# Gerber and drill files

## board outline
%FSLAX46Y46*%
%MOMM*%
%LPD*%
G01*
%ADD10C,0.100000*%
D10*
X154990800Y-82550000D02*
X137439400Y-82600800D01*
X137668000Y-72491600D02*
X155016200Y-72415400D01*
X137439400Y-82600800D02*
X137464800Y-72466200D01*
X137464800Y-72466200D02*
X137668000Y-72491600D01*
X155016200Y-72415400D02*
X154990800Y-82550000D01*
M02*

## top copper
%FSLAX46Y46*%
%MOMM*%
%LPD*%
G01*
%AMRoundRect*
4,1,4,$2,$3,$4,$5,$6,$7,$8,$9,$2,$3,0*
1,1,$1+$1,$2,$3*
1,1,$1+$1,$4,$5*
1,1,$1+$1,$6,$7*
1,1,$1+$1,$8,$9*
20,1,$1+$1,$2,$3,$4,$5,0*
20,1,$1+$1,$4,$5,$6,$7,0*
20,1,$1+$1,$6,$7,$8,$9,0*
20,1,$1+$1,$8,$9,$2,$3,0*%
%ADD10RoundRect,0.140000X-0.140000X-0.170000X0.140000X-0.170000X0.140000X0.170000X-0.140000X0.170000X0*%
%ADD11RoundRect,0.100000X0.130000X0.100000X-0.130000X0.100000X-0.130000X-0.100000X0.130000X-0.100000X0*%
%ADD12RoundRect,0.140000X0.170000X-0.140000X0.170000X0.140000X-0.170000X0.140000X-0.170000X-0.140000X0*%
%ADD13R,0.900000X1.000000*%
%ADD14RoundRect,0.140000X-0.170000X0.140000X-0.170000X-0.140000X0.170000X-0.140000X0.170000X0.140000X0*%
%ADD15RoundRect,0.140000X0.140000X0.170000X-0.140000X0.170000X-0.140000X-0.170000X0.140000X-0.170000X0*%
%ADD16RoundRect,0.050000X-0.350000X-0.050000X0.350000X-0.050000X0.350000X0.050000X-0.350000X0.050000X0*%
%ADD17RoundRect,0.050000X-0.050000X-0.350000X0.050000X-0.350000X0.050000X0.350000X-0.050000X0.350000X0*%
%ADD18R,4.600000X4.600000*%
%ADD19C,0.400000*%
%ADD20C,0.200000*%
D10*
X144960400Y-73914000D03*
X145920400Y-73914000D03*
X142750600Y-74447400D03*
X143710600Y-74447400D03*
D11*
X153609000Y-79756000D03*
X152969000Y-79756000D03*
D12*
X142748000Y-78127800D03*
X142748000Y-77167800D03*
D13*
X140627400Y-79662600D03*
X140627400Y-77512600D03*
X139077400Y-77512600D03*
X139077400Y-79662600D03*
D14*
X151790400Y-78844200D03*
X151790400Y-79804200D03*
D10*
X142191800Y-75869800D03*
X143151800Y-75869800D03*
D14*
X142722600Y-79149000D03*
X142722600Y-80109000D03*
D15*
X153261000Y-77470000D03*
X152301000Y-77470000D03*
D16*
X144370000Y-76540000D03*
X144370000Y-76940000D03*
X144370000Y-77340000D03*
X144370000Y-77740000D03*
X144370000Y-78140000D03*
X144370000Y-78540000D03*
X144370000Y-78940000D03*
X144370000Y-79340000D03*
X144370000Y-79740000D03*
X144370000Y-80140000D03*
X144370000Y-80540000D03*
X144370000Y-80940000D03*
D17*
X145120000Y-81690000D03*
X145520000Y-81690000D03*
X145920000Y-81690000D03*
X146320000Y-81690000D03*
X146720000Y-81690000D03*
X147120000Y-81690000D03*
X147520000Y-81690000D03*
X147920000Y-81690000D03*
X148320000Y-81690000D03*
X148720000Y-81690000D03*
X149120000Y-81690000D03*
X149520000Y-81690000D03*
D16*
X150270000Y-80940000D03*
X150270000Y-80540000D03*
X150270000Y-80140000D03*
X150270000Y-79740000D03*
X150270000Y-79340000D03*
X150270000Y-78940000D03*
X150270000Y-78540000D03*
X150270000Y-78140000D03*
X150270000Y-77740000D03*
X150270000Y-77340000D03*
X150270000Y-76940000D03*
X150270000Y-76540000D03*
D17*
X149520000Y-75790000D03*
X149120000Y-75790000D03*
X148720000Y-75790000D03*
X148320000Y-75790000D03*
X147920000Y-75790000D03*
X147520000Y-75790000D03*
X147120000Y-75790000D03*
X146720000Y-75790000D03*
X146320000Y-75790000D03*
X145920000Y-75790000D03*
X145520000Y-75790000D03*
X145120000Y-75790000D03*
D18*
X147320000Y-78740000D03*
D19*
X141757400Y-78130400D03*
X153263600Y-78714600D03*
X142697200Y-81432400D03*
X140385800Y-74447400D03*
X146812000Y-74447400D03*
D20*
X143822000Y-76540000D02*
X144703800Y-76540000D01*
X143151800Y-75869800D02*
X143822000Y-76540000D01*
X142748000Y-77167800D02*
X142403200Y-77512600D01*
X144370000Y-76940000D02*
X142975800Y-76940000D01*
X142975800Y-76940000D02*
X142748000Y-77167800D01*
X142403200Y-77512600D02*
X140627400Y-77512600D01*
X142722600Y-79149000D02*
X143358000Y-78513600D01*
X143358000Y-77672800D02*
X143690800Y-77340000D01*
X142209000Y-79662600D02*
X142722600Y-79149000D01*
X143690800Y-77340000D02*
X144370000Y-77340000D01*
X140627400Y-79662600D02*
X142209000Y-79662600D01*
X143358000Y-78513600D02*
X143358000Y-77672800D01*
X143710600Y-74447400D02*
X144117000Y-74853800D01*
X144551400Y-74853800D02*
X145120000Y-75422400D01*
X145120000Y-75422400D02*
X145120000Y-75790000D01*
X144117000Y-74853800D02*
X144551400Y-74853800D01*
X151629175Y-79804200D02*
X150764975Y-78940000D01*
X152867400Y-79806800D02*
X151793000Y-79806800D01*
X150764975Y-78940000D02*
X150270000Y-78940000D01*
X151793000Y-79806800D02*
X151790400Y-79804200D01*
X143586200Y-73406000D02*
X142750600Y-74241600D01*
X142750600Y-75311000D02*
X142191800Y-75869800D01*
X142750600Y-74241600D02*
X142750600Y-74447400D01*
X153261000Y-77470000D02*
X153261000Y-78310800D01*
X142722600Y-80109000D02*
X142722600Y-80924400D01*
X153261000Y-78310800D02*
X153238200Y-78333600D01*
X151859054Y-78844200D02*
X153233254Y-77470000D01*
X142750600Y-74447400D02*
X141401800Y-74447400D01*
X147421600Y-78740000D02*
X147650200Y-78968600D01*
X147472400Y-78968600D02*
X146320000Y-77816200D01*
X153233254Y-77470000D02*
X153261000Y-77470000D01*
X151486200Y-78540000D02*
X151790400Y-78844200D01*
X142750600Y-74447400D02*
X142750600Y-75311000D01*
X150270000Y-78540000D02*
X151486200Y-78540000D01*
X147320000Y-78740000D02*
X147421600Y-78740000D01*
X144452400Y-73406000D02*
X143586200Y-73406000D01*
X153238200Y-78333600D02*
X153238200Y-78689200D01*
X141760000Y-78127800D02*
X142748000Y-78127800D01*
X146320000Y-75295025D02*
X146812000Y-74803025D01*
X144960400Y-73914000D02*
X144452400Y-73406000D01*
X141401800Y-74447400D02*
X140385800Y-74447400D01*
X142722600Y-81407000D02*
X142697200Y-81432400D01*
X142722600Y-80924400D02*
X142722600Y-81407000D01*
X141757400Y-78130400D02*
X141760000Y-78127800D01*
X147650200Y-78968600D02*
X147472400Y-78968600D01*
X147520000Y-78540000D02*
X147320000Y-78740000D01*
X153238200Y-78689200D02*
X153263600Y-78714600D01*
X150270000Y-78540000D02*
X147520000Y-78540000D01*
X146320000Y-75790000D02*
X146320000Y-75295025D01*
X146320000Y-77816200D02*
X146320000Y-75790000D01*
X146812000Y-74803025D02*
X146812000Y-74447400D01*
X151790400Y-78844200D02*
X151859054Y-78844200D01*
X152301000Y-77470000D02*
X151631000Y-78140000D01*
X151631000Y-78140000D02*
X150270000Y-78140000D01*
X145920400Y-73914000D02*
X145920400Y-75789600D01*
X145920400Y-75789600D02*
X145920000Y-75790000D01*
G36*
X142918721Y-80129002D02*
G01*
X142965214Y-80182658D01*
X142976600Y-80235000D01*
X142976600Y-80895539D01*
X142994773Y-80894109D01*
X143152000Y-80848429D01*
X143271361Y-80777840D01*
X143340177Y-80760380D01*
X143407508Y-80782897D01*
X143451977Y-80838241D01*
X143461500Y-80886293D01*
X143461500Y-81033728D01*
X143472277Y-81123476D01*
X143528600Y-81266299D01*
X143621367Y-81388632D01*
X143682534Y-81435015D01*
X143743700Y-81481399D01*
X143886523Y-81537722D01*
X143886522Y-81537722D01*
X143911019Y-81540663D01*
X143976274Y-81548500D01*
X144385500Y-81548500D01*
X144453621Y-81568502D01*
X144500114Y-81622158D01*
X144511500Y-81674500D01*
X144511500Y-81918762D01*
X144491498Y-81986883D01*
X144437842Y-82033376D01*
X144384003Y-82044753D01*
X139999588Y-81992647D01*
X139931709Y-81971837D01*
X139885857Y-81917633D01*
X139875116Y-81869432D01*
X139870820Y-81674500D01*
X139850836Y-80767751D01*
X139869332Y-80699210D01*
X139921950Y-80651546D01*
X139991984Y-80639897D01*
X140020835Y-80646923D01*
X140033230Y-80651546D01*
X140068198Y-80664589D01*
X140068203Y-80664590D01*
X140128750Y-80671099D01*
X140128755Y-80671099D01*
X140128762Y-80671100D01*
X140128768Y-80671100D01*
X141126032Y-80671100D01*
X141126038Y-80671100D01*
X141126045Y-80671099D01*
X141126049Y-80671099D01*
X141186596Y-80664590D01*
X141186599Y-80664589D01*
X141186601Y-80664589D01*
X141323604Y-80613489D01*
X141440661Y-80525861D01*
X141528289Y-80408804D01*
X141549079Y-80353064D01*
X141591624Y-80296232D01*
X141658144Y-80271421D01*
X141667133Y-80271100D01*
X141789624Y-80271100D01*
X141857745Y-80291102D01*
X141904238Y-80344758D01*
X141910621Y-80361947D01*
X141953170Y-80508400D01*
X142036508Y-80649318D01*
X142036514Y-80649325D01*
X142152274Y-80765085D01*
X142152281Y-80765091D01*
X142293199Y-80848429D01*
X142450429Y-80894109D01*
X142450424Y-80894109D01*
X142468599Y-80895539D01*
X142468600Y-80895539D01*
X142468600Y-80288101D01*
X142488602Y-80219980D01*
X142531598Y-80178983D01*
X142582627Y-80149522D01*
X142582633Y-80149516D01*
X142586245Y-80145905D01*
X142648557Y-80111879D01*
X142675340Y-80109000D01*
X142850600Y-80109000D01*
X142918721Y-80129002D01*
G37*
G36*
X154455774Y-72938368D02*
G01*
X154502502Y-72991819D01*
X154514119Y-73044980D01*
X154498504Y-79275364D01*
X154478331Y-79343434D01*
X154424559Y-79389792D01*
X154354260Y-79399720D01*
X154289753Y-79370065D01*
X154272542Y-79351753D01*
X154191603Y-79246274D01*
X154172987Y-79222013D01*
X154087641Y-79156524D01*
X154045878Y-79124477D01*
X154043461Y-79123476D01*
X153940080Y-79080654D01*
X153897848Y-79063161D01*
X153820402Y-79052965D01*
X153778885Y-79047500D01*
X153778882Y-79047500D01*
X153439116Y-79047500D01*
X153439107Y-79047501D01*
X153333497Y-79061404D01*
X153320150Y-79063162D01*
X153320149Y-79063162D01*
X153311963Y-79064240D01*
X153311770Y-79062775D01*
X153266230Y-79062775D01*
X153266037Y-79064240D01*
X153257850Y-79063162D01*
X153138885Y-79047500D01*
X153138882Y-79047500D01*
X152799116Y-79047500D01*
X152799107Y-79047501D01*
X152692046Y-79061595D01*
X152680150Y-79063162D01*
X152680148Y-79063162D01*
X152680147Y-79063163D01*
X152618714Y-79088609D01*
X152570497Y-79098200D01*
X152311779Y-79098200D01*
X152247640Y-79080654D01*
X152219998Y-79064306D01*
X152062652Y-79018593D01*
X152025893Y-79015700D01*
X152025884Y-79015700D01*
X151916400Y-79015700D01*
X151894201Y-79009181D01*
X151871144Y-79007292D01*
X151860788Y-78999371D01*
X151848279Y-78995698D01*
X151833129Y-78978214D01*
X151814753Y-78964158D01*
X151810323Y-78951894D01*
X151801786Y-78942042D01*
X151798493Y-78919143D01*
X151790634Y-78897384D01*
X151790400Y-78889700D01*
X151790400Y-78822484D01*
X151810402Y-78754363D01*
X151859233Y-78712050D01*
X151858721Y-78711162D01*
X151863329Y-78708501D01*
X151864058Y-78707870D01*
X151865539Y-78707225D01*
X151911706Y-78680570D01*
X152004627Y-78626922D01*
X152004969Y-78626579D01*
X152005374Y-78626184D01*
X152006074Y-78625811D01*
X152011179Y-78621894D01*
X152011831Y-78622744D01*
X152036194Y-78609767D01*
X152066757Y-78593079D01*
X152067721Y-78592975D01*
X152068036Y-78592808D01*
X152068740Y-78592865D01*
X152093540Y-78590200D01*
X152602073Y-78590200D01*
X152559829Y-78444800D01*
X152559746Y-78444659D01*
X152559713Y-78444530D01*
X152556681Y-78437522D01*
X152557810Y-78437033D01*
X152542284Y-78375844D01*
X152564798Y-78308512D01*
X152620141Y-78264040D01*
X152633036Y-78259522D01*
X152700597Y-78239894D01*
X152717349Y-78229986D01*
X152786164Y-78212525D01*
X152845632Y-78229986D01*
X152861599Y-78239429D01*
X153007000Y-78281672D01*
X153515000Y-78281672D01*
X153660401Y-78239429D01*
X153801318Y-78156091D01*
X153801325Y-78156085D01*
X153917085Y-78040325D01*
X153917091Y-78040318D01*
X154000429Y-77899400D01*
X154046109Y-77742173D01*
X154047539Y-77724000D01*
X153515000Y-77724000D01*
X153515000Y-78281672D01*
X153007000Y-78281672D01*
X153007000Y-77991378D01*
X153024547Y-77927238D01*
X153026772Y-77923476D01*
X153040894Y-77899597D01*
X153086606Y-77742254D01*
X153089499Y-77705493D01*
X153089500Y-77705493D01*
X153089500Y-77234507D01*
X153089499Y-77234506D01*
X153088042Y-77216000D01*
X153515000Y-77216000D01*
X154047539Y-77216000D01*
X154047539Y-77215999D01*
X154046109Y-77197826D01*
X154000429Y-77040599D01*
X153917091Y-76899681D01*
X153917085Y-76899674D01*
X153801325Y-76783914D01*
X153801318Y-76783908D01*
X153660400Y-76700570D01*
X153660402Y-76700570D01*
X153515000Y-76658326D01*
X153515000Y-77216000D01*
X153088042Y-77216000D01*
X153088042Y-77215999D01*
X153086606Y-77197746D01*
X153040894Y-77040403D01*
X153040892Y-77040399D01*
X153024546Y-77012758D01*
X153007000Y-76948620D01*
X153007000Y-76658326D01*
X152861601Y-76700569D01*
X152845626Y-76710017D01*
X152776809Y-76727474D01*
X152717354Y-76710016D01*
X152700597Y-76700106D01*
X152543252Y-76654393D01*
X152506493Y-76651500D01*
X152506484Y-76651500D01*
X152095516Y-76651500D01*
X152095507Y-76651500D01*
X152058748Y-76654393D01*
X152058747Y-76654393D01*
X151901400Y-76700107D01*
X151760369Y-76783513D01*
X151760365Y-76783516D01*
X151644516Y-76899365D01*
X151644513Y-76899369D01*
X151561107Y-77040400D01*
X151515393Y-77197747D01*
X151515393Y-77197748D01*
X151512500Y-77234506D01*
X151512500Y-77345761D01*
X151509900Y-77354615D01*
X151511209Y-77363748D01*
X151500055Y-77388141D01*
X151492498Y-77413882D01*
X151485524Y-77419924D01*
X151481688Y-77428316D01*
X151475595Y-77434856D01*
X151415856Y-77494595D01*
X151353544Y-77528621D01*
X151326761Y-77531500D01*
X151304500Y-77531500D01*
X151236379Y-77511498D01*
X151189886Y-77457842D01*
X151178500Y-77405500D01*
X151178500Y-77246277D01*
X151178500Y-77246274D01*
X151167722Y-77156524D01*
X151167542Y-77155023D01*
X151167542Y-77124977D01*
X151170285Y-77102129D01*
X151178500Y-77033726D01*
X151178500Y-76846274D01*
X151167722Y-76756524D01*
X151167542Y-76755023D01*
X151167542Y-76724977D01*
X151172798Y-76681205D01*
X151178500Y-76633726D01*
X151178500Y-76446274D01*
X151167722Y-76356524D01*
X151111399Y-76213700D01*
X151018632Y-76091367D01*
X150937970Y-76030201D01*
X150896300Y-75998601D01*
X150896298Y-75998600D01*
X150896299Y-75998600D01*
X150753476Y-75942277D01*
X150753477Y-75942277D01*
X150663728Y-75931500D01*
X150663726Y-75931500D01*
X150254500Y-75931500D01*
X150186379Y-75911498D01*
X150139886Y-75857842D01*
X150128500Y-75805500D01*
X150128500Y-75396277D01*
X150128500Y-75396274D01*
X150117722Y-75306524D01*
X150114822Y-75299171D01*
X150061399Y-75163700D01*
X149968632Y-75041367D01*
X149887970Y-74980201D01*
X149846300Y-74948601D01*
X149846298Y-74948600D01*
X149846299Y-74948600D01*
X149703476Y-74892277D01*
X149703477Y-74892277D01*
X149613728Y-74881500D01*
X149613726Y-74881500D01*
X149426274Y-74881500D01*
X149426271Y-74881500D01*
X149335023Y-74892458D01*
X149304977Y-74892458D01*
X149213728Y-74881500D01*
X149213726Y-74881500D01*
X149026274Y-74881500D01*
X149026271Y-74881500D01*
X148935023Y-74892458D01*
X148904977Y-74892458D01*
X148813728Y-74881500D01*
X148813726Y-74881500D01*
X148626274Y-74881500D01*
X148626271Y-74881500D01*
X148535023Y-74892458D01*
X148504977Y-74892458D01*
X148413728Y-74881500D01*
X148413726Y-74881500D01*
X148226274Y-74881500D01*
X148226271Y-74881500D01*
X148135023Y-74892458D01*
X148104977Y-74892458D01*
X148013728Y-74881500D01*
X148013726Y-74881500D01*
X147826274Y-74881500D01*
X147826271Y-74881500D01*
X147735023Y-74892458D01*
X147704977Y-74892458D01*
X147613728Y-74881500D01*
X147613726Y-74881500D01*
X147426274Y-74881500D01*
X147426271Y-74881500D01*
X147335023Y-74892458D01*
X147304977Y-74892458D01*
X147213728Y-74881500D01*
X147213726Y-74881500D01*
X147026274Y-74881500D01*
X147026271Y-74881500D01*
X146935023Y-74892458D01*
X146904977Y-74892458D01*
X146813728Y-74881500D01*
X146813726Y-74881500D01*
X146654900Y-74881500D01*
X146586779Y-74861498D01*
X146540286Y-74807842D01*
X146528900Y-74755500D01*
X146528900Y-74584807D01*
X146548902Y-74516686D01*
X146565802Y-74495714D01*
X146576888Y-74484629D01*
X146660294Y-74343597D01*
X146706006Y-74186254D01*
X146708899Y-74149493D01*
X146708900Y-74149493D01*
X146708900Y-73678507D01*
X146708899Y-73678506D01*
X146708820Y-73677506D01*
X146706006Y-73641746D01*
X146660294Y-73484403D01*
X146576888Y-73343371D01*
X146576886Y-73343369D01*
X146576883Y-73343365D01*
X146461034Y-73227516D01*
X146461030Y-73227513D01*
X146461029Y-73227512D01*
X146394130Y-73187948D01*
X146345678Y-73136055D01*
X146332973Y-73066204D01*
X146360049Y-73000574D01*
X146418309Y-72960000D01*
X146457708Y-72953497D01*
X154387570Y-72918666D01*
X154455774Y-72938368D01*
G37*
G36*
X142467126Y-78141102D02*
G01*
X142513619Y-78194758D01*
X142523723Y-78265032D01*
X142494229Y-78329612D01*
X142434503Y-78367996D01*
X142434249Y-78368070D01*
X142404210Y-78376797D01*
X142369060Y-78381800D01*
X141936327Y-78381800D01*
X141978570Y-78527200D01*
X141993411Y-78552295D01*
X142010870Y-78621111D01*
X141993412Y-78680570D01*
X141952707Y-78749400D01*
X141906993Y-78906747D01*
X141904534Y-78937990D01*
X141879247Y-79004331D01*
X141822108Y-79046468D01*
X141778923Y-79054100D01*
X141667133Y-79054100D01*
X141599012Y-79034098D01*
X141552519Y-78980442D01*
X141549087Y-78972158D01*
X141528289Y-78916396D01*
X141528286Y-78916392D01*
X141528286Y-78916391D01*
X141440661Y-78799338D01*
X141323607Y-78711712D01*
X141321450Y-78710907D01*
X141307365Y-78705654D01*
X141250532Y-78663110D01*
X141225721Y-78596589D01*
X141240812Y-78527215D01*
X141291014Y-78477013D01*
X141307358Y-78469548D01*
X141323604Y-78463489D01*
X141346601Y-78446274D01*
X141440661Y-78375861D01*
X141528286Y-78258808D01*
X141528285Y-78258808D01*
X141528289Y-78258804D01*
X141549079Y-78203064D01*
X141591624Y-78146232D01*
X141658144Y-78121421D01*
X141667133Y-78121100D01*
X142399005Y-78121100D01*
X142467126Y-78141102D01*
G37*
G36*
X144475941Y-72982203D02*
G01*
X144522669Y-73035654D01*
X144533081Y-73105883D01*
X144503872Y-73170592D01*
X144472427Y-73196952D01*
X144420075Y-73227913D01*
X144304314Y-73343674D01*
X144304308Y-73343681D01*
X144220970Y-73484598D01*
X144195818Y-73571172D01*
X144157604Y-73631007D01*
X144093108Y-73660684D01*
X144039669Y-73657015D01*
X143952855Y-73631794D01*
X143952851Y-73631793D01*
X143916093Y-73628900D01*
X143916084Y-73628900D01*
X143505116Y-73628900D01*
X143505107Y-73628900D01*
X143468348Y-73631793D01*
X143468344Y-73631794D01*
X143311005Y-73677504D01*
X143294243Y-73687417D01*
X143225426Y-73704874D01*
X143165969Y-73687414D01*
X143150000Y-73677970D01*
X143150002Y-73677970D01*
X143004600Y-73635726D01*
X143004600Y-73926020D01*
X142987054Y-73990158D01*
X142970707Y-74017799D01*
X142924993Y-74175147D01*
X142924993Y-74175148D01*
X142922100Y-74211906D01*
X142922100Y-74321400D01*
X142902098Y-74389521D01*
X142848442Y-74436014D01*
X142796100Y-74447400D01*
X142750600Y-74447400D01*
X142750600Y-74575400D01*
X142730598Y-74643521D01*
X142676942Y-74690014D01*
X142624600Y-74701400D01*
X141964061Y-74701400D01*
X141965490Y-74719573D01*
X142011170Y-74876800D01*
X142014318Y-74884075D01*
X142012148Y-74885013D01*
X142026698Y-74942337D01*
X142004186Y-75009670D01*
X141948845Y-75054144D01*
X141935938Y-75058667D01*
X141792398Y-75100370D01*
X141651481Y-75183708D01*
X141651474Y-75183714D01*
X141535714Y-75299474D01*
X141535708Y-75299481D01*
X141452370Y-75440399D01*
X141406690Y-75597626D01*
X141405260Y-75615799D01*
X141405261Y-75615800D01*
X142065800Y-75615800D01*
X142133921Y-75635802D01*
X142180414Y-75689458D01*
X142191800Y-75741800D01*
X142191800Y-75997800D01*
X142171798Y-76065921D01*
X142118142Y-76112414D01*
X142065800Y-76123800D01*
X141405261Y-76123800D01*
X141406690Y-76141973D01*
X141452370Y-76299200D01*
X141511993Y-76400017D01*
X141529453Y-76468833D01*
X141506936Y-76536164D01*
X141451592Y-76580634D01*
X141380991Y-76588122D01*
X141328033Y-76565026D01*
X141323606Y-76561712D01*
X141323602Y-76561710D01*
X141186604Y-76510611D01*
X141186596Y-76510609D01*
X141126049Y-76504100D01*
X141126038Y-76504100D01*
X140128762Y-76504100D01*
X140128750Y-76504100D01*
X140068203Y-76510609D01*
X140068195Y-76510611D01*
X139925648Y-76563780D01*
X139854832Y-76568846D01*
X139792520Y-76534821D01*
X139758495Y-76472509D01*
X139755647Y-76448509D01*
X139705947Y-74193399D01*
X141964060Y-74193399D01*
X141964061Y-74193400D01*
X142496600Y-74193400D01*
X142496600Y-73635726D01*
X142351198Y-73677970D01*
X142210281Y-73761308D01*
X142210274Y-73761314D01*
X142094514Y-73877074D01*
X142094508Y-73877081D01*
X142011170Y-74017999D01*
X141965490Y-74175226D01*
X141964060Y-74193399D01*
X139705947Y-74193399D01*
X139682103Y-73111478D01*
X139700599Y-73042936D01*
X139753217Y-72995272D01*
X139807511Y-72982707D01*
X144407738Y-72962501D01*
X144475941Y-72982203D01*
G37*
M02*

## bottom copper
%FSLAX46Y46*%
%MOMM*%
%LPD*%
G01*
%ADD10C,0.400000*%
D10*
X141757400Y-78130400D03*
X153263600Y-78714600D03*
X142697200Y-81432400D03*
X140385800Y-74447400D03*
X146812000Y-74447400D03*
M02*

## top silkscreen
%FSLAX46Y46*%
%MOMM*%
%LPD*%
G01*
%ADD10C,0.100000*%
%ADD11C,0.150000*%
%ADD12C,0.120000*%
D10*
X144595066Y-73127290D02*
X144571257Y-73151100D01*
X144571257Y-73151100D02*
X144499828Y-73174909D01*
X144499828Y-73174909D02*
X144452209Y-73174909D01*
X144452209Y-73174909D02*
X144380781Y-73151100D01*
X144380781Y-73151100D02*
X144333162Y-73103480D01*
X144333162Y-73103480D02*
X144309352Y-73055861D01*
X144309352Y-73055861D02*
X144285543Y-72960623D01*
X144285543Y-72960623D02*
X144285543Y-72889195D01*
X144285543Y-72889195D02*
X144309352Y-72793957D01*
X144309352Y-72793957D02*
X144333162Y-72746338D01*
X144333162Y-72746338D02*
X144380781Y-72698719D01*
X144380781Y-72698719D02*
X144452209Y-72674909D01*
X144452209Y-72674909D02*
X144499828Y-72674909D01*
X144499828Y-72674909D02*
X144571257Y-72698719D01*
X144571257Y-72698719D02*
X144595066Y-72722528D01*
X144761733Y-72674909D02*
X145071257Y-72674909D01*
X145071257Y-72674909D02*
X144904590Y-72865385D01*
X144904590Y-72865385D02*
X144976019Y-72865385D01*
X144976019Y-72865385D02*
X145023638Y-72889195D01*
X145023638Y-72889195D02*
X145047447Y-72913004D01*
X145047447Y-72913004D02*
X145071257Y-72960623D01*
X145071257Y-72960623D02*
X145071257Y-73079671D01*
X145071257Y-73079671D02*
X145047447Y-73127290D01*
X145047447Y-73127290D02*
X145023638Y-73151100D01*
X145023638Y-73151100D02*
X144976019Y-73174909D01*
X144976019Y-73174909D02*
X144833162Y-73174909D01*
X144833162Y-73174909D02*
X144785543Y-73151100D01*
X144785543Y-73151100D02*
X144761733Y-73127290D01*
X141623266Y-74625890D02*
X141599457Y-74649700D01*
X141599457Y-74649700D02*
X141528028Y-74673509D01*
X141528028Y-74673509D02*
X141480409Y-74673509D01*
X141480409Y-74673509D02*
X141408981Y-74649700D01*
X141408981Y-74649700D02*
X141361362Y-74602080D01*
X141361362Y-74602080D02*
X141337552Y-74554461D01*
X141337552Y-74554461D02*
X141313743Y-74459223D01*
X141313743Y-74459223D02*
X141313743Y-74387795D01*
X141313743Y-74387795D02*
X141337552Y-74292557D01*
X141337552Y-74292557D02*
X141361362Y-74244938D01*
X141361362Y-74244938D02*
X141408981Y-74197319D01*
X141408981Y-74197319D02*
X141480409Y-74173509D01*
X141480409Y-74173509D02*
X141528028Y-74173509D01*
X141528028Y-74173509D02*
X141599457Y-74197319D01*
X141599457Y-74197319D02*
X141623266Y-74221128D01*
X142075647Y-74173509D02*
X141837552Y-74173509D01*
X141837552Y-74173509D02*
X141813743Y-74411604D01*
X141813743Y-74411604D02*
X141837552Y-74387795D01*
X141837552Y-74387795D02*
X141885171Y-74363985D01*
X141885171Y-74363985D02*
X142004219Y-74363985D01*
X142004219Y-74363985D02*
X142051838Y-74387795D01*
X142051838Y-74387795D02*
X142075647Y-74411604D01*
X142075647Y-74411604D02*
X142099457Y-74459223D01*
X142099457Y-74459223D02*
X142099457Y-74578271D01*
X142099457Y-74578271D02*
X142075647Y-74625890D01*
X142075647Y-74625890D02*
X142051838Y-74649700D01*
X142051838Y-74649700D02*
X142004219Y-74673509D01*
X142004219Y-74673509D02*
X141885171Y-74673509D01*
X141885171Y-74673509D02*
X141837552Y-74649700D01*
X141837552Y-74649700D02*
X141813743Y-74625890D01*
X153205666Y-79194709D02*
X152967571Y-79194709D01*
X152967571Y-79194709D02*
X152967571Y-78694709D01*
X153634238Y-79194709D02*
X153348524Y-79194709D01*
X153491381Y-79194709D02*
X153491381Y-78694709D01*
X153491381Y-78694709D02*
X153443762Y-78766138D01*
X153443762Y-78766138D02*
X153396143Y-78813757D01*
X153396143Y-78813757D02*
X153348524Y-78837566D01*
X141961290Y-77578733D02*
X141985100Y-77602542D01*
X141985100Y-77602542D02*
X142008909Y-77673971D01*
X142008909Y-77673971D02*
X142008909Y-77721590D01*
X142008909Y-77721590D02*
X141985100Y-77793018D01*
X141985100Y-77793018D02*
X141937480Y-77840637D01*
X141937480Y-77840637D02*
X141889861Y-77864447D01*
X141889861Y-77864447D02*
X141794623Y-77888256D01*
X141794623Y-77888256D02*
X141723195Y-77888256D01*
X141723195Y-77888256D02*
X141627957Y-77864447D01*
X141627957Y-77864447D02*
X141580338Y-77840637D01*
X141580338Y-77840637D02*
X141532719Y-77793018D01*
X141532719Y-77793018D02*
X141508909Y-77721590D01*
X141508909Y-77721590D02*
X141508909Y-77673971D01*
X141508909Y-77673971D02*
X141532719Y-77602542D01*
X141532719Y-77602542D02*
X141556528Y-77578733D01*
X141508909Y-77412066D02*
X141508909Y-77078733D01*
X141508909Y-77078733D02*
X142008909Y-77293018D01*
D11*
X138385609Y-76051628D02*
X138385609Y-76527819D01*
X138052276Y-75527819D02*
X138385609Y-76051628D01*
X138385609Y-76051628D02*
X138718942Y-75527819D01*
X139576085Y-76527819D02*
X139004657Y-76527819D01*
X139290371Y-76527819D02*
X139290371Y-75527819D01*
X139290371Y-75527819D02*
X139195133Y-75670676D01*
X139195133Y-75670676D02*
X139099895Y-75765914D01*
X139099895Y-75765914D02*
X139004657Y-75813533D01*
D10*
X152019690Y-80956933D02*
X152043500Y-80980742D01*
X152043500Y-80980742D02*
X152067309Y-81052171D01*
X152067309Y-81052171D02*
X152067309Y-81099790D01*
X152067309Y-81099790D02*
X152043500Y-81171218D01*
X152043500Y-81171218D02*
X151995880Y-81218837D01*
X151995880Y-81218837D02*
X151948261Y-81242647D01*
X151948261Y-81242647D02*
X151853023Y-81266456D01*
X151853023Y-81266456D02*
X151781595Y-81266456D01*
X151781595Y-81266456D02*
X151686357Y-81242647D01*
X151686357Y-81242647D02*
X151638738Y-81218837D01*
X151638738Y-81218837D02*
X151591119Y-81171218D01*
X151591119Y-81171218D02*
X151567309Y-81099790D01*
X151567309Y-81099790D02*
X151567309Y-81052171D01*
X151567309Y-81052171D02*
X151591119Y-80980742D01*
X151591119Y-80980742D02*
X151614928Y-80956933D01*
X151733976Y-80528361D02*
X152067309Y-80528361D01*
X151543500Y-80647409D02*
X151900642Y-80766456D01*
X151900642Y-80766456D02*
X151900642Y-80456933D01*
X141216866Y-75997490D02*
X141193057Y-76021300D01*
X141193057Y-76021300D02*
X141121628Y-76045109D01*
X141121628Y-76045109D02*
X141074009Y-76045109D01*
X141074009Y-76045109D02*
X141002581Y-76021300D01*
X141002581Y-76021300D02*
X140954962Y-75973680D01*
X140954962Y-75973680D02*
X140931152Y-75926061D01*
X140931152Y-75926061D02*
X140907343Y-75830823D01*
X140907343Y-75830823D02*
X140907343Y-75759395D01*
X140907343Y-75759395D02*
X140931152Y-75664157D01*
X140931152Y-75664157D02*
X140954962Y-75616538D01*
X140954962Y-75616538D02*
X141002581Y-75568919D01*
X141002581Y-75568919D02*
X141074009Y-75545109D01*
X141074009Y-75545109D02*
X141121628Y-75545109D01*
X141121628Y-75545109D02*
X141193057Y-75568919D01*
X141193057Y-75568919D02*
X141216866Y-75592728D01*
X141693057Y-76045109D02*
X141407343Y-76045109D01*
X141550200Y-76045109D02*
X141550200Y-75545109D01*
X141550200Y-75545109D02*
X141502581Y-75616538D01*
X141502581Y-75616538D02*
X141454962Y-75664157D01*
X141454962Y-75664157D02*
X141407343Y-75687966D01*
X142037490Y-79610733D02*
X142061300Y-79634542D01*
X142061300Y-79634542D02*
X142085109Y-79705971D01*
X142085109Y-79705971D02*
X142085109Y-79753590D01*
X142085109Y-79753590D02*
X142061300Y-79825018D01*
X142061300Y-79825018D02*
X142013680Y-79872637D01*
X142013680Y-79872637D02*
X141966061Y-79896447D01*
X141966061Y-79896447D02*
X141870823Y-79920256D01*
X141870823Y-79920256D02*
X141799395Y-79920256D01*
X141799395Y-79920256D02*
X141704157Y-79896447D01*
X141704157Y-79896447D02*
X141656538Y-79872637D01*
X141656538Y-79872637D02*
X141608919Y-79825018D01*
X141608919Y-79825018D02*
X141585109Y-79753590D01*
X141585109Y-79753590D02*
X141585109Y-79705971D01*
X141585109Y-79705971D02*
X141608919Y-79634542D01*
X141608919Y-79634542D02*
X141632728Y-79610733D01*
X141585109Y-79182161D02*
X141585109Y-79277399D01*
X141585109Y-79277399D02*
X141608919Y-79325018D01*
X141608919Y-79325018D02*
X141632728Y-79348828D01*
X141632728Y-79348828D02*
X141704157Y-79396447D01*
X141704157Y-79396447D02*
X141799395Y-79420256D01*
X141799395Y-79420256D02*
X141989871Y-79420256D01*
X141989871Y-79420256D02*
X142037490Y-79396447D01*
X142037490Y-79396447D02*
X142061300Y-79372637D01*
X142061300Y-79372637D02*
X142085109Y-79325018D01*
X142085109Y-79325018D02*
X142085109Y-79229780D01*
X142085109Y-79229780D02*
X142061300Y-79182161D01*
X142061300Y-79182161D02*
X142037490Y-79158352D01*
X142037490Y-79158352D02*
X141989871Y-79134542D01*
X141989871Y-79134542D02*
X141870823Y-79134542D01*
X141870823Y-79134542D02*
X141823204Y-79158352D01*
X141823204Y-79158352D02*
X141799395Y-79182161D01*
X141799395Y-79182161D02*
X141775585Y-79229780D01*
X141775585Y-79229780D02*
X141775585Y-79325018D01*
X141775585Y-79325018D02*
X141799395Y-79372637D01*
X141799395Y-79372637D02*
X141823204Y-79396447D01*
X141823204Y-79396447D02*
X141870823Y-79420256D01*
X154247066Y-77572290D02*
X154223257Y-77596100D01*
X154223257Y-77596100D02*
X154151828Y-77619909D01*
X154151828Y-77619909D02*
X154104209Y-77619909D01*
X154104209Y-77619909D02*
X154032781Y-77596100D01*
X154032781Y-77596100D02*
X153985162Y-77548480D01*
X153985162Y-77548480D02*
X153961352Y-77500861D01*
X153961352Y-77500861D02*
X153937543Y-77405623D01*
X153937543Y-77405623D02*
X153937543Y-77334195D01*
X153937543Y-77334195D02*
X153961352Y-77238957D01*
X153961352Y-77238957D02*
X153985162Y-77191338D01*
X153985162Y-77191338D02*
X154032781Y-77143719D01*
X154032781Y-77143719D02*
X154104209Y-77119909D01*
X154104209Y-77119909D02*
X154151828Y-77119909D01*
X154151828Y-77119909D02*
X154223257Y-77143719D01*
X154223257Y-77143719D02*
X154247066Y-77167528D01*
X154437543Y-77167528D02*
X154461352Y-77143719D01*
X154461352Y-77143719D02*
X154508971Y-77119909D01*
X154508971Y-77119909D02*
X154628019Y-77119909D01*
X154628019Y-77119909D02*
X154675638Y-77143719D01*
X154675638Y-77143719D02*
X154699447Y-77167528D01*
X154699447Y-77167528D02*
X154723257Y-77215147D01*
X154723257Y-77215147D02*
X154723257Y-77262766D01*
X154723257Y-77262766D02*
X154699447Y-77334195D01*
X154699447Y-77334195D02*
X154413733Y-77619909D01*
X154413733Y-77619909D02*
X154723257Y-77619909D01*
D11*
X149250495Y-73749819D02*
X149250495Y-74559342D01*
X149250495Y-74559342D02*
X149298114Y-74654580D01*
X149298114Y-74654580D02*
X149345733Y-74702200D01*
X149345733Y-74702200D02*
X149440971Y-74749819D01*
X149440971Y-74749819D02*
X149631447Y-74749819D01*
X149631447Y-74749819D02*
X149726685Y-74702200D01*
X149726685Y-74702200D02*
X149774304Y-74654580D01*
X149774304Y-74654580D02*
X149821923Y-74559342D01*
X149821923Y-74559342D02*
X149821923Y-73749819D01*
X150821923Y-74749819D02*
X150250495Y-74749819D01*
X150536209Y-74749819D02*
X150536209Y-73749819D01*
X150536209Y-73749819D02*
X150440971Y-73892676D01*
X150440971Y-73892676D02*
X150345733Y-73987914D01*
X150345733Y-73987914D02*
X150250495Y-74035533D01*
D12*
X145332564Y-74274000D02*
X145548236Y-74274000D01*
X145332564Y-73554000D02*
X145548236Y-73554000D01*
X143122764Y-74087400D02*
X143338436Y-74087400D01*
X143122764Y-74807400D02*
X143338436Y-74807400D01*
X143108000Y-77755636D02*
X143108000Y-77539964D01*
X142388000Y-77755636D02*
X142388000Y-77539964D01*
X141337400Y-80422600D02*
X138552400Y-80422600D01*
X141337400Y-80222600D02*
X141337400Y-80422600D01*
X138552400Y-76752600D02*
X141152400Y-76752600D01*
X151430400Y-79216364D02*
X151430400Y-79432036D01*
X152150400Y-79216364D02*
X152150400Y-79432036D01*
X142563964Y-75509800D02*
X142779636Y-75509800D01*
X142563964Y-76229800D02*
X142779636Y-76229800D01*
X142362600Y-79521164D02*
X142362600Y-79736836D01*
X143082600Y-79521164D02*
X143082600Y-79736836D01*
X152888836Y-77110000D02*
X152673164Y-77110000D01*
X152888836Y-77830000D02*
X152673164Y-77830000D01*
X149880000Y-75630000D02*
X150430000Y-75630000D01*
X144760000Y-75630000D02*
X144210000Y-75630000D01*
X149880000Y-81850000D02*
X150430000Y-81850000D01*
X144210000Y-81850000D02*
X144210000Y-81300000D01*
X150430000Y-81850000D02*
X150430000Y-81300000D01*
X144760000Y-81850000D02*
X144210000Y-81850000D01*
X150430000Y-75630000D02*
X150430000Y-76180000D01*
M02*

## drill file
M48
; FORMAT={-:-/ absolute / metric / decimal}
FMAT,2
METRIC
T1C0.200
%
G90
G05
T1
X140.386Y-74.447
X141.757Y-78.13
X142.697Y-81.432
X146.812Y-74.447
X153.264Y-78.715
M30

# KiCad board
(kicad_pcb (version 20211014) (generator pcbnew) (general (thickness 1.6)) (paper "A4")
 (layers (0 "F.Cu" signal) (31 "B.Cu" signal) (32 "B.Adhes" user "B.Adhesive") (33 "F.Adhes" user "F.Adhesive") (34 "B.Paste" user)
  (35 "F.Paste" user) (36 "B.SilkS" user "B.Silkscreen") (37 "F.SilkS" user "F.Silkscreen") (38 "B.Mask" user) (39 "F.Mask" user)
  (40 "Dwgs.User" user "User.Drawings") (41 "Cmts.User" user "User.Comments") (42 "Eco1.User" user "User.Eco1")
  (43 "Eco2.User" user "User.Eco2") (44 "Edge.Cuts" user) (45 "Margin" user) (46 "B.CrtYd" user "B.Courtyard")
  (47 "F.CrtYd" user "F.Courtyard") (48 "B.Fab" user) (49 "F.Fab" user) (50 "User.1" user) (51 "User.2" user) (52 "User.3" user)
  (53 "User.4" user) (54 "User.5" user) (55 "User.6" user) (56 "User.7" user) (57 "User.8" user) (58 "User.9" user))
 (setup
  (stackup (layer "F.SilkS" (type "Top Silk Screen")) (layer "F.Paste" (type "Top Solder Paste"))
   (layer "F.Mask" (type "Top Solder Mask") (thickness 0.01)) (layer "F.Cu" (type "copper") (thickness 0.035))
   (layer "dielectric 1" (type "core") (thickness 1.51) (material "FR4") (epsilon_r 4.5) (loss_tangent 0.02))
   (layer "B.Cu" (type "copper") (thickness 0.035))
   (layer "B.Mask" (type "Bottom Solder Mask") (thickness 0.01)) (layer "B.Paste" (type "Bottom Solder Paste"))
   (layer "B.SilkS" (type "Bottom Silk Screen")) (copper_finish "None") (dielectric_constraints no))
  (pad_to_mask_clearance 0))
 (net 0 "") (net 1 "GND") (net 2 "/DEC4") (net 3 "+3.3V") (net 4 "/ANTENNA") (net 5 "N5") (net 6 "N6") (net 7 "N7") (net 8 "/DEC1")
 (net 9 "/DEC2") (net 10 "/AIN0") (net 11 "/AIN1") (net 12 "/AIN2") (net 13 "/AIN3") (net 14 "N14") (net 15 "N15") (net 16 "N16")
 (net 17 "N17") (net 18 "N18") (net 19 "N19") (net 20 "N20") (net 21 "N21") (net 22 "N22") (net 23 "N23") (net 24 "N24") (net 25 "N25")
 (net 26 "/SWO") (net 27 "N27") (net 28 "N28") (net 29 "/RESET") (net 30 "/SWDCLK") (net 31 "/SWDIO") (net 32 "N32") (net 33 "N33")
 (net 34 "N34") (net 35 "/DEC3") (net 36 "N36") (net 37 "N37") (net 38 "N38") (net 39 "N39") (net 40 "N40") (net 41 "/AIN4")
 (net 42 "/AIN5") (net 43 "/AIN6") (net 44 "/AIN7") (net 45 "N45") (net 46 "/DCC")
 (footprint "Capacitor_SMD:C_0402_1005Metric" (layer "F.Cu") (at 145.4404 73.914)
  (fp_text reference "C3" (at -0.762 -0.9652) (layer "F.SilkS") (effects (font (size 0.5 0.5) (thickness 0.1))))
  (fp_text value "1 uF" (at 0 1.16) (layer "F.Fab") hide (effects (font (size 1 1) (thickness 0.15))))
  (fp_line (start -0.107836 0.36) (end 0.107836 0.36) (layer "F.SilkS") (width 0.12))
  (fp_line (start -0.107836 -0.36) (end 0.107836 -0.36) (layer "F.SilkS") (width 0.12))
  (pad "1" smd roundrect (at -0.48 0) (size 0.56 0.62) (layers "F.Cu" "F.Paste" "F.Mask") (roundrect_rratio 0.25) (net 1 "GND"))
  (pad "2" smd roundrect (at 0.48 0) (size 0.56 0.62) (layers "F.Cu" "F.Paste" "F.Mask") (roundrect_rratio 0.25) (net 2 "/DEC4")))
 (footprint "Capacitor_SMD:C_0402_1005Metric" (layer "F.Cu") (at 143.2306 74.4474)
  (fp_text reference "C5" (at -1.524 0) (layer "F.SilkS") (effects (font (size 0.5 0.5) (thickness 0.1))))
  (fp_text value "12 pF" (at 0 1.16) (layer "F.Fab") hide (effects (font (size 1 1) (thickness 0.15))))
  (fp_line (start -0.107836 -0.36) (end 0.107836 -0.36) (layer "F.SilkS") (width 0.12))
  (fp_line (start -0.107836 0.36) (end 0.107836 0.36) (layer "F.SilkS") (width 0.12))
  (pad "1" smd roundrect (at -0.48 0) (size 0.56 0.62) (layers "F.Cu" "F.Paste" "F.Mask") (roundrect_rratio 0.25) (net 1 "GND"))
  (pad "2" smd roundrect (at 0.48 0) (size 0.56 0.62) (layers "F.Cu" "F.Paste" "F.Mask") (roundrect_rratio 0.25) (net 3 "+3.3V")))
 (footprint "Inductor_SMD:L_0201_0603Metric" (layer "F.Cu") (at 153.289 79.756 180)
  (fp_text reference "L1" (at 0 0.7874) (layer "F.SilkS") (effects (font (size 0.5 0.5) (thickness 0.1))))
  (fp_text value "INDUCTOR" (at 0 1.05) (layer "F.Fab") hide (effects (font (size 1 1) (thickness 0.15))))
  (pad "" smd roundrect (at -0.345 0 180) (size 0.318 0.36) (layers "F.Paste") (roundrect_rratio 0.25))
  (pad "" smd roundrect (at 0.345 0 180) (size 0.318 0.36) (layers "F.Paste") (roundrect_rratio 0.25))
  (pad "1" smd roundrect (at -0.32 0 180) (size 0.46 0.4) (layers "F.Cu" "F.Mask") (roundrect_rratio 0.25) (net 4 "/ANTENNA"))
  (pad "2" smd roundrect (at 0.32 0 180) (size 0.46 0.4) (layers "F.Cu" "F.Mask") (roundrect_rratio 0.25) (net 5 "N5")))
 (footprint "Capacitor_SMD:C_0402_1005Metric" (layer "F.Cu") (at 142.748 77.6478 90)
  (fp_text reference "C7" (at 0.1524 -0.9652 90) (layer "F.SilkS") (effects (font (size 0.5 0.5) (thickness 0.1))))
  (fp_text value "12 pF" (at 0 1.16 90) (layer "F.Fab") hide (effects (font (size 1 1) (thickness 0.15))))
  (fp_line (start -0.107836 0.36) (end 0.107836 0.36) (layer "F.SilkS") (width 0.12))
  (fp_line (start -0.107836 -0.36) (end 0.107836 -0.36) (layer "F.SilkS") (width 0.12))
  (pad "1" smd roundrect (at -0.48 0 90) (size 0.56 0.62) (layers "F.Cu" "F.Paste" "F.Mask") (roundrect_rratio 0.25) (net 1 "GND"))
  (pad "2" smd roundrect (at 0.48 0 90) (size 0.56 0.62) (layers "F.Cu" "F.Paste" "F.Mask") (roundrect_rratio 0.25) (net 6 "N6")))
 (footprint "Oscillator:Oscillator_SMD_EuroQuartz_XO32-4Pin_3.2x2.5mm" (layer "F.Cu") (at 139.8524 78.5876 180)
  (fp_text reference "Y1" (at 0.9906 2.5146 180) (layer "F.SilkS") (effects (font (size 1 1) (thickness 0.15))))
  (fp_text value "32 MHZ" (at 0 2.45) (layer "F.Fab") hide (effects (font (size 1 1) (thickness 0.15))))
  (fp_line (start -1.485 -1.835) (end 1.3 -1.835) (layer "F.SilkS") (width 0.12))
  (fp_line (start -1.485 -1.635) (end -1.485 -1.835) (layer "F.SilkS") (width 0.12))
  (fp_line (start 1.3 1.835) (end -1.3 1.835) (layer "F.SilkS") (width 0.12))
  (pad "1" smd rect (at -0.775 -1.075 90) (size 1 0.9) (layers "F.Cu" "F.Paste" "F.Mask") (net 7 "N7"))
  (pad "2" smd rect (at -0.775 1.075 90) (size 1 0.9) (layers "F.Cu" "F.Paste" "F.Mask") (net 6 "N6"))
  (pad "3" smd rect (at 0.775 1.075 90) (size 1 0.9) (layers "F.Cu" "F.Paste" "F.Mask"))
  (pad "4" smd rect (at 0.775 -1.075 90) (size 1 0.9) (layers "F.Cu" "F.Paste" "F.Mask")))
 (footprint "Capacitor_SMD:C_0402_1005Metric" (layer "F.Cu") (at 151.7904 79.3242 -90)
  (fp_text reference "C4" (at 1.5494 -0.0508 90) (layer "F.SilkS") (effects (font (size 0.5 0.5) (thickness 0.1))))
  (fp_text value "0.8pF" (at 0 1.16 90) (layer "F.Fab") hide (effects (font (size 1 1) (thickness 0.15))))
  (fp_line (start -0.107836 0.36) (end 0.107836 0.36) (layer "F.SilkS") (width 0.12))
  (fp_line (start -0.107836 -0.36) (end 0.107836 -0.36) (layer "F.SilkS") (width 0.12))
  (pad "1" smd roundrect (at -0.48 0 270) (size 0.56 0.62) (layers "F.Cu" "F.Paste" "F.Mask") (roundrect_rratio 0.25) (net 1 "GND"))
  (pad "2" smd roundrect (at 0.48 0 270) (size 0.56 0.62) (layers "F.Cu" "F.Paste" "F.Mask") (roundrect_rratio 0.25) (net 5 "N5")))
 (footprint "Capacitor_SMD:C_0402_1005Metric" (layer "F.Cu") (at 142.6718 75.8698)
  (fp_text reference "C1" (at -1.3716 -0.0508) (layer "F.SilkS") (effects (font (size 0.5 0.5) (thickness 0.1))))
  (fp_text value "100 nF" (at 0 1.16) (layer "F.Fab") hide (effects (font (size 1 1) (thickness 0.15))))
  (fp_line (start -0.107836 -0.36) (end 0.107836 -0.36) (layer "F.SilkS") (width 0.12))
  (fp_line (start -0.107836 0.36) (end 0.107836 0.36) (layer "F.SilkS") (width 0.12))
  (pad "1" smd roundrect (at -0.48 0) (size 0.56 0.62) (layers "F.Cu" "F.Paste" "F.Mask") (roundrect_rratio 0.25) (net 1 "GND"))
  (pad "2" smd roundrect (at 0.48 0) (size 0.56 0.62) (layers "F.Cu" "F.Paste" "F.Mask") (roundrect_rratio 0.25) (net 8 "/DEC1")))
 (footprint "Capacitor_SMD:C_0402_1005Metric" (layer "F.Cu") (at 142.7226 79.629 -90)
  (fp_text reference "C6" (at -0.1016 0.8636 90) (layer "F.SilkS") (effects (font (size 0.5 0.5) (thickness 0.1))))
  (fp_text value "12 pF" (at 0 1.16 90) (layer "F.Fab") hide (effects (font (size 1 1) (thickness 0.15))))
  (fp_line (start -0.107836 0.36) (end 0.107836 0.36) (layer "F.SilkS") (width 0.12))
  (fp_line (start -0.107836 -0.36) (end 0.107836 -0.36) (layer "F.SilkS") (width 0.12))
  (pad "1" smd roundrect (at -0.48 0 270) (size 0.56 0.62) (layers "F.Cu" "F.Paste" "F.Mask") (roundrect_rratio 0.25) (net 7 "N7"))
  (pad "2" smd roundrect (at 0.48 0 270) (size 0.56 0.62) (layers "F.Cu" "F.Paste" "F.Mask") (roundrect_rratio 0.25) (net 1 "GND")))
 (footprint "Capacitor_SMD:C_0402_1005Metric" (layer "F.Cu") (at 152.781 77.47 180)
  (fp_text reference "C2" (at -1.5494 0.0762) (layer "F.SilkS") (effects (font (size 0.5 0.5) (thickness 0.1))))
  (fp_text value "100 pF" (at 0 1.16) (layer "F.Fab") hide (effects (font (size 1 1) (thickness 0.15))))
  (fp_line (start -0.107836 0.36) (end 0.107836 0.36) (layer "F.SilkS") (width 0.12))
  (fp_line (start -0.107836 -0.36) (end 0.107836 -0.36) (layer "F.SilkS") (width 0.12))
  (pad "1" smd roundrect (at -0.48 0 180) (size 0.56 0.62) (layers "F.Cu" "F.Paste" "F.Mask") (roundrect_rratio 0.25) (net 1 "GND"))
  (pad "2" smd roundrect (at 0.48 0 180) (size 0.56 0.62) (layers "F.Cu" "F.Paste" "F.Mask") (roundrect_rratio 0.25) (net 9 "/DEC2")))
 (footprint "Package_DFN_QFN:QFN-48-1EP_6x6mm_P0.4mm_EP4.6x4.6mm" (layer "F.Cu") (at 147.32 78.74)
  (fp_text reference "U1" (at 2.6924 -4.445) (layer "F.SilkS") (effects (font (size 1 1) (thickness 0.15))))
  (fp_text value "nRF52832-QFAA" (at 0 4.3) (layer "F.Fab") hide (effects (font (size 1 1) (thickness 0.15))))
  (fp_line (start 2.56 -3.11) (end 3.11 -3.11) (layer "F.SilkS") (width 0.12))
  (fp_line (start -2.56 -3.11) (end -3.11 -3.11) (layer "F.SilkS") (width 0.12))
  (fp_line (start 2.56 3.11) (end 3.11 3.11) (layer "F.SilkS") (width 0.12))
  (fp_line (start -3.11 3.11) (end -3.11 2.56) (layer "F.SilkS") (width 0.12))
  (fp_line (start 3.11 3.11) (end 3.11 2.56) (layer "F.SilkS") (width 0.12))
  (fp_line (start -2.56 3.11) (end -3.11 3.11) (layer "F.SilkS") (width 0.12))
  (fp_line (start 3.11 -3.11) (end 3.11 -2.56) (layer "F.SilkS") (width 0.12))
  (pad "" smd roundrect (at 0 1.53) (size 1.24 1.24) (layers "F.Paste") (roundrect_rratio 0.201613))
  (pad "" smd roundrect (at 1.53 -1.53) (size 1.24 1.24) (layers "F.Paste") (roundrect_rratio 0.201613))
  (pad "" smd roundrect (at 1.53 0) (size 1.24 1.24) (layers "F.Paste") (roundrect_rratio 0.201613))
  (pad "" smd roundrect (at 0 0) (size 1.24 1.24) (layers "F.Paste") (roundrect_rratio 0.201613))
  (pad "" smd roundrect (at -1.53 0) (size 1.24 1.24) (layers "F.Paste") (roundrect_rratio 0.201613))
  (pad "" smd roundrect (at 1.53 1.53) (size 1.24 1.24) (layers "F.Paste") (roundrect_rratio 0.201613))
  (pad "" smd roundrect (at 0 -1.53) (size 1.24 1.24) (layers "F.Paste") (roundrect_rratio 0.201613))
  (pad "" smd roundrect (at -1.53 -1.53) (size 1.24 1.24) (layers "F.Paste") (roundrect_rratio 0.201613))
  (pad "" smd roundrect (at -1.53 1.53) (size 1.24 1.24) (layers "F.Paste") (roundrect_rratio 0.201613))
  (pad "1" smd roundrect (at -2.95 -2.2) (size 0.8 0.2) (layers "F.Cu" "F.Paste" "F.Mask") (roundrect_rratio 0.25) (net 8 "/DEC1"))
  (pad "2" smd roundrect (at -2.95 -1.8) (size 0.8 0.2) (layers "F.Cu" "F.Paste" "F.Mask") (roundrect_rratio 0.25) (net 6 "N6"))
  (pad "3" smd roundrect (at -2.95 -1.4) (size 0.8 0.2) (layers "F.Cu" "F.Paste" "F.Mask") (roundrect_rratio 0.25) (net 7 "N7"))
  (pad "4" smd roundrect (at -2.95 -1) (size 0.8 0.2) (layers "F.Cu" "F.Paste" "F.Mask") (roundrect_rratio 0.25) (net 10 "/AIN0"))
  (pad "5" smd roundrect (at -2.95 -0.6) (size 0.8 0.2) (layers "F.Cu" "F.Paste" "F.Mask") (roundrect_rratio 0.25) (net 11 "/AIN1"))
  (pad "6" smd roundrect (at -2.95 -0.2) (size 0.8 0.2) (layers "F.Cu" "F.Paste" "F.Mask") (roundrect_rratio 0.25) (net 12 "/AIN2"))
  (pad "7" smd roundrect (at -2.95 0.2) (size 0.8 0.2) (layers "F.Cu" "F.Paste" "F.Mask") (roundrect_rratio 0.25) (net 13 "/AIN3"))
  (pad "8" smd roundrect (at -2.95 0.6) (size 0.8 0.2) (layers "F.Cu" "F.Paste" "F.Mask") (roundrect_rratio 0.25) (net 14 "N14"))
  (pad "9" smd roundrect (at -2.95 1) (size 0.8 0.2) (layers "F.Cu" "F.Paste" "F.Mask") (roundrect_rratio 0.25) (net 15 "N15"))
  (pad "10" smd roundrect (at -2.95 1.4) (size 0.8 0.2) (layers "F.Cu" "F.Paste" "F.Mask") (roundrect_rratio 0.25) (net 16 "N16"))
  (pad "11" smd roundrect (at -2.95 1.8) (size 0.8 0.2) (layers "F.Cu" "F.Paste" "F.Mask") (roundrect_rratio 0.25) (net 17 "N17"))
  (pad "12" smd roundrect (at -2.95 2.2) (size 0.8 0.2) (layers "F.Cu" "F.Paste" "F.Mask") (roundrect_rratio 0.25) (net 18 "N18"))
  (pad "13" smd roundrect (at -2.2 2.95) (size 0.2 0.8) (layers "F.Cu" "F.Paste" "F.Mask") (roundrect_rratio 0.25) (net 3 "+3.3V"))
  (pad "14" smd roundrect (at -1.8 2.95) (size 0.2 0.8) (layers "F.Cu" "F.Paste" "F.Mask") (roundrect_rratio 0.25) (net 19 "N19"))
  (pad "15" smd roundrect (at -1.4 2.95) (size 0.2 0.8) (layers "F.Cu" "F.Paste" "F.Mask") (roundrect_rratio 0.25) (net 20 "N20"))
  (pad "16" smd roundrect (at -1 2.95) (size 0.2 0.8) (layers "F.Cu" "F.Paste" "F.Mask") (roundrect_rratio 0.25) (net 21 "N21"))
  (pad "17" smd roundrect (at -0.6 2.95) (size 0.2 0.8) (layers "F.Cu" "F.Paste" "F.Mask") (roundrect_rratio 0.25) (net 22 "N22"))
  (pad "18" smd roundrect (at -0.2 2.95) (size 0.2 0.8) (layers "F.Cu" "F.Paste" "F.Mask") (roundrect_rratio 0.25) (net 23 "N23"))
  (pad "19" smd roundrect (at 0.2 2.95) (size 0.2 0.8) (layers "F.Cu" "F.Paste" "F.Mask") (roundrect_rratio 0.25) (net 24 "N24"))
  (pad "20" smd roundrect (at 0.6 2.95) (size 0.2 0.8) (layers "F.Cu" "F.Paste" "F.Mask") (roundrect_rratio 0.25) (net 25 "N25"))
  (pad "21" smd roundrect (at 1 2.95) (size 0.2 0.8) (layers "F.Cu" "F.Paste" "F.Mask") (roundrect_rratio 0.25) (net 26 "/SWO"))
  (pad "22" smd roundrect (at 1.4 2.95) (size 0.2 0.8) (layers "F.Cu" "F.Paste" "F.Mask") (roundrect_rratio 0.25) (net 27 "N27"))
  (pad "23" smd roundrect (at 1.8 2.95) (size 0.2 0.8) (layers "F.Cu" "F.Paste" "F.Mask") (roundrect_rratio 0.25) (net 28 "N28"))
  (pad "24" smd roundrect (at 2.2 2.95) (size 0.2 0.8) (layers "F.Cu" "F.Paste" "F.Mask") (roundrect_rratio 0.25) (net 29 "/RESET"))
  (pad "25" smd roundrect (at 2.95 2.2) (size 0.8 0.2) (layers "F.Cu" "F.Paste" "F.Mask") (roundrect_rratio 0.25) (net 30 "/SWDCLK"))
  (pad "26" smd roundrect (at 2.95 1.8) (size 0.8 0.2) (layers "F.Cu" "F.Paste" "F.Mask") (roundrect_rratio 0.25) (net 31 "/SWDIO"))
  (pad "27" smd roundrect (at 2.95 1.4) (size 0.8 0.2) (layers "F.Cu" "F.Paste" "F.Mask") (roundrect_rratio 0.25) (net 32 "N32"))
  (pad "28" smd roundrect (at 2.95 1) (size 0.8 0.2) (layers "F.Cu" "F.Paste" "F.Mask") (roundrect_rratio 0.25) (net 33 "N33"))
  (pad "29" smd roundrect (at 2.95 0.6) (size 0.8 0.2) (layers "F.Cu" "F.Paste" "F.Mask") (roundrect_rratio 0.25) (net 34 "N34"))
  (pad "30" smd roundrect (at 2.95 0.2) (size 0.8 0.2) (layers "F.Cu" "F.Paste" "F.Mask") (roundrect_rratio 0.25) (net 5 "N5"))
  (pad "31" smd roundrect (at 2.95 -0.2) (size 0.8 0.2) (layers "F.Cu" "F.Paste" "F.Mask") (roundrect_rratio 0.25) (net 1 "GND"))
  (pad "32" smd roundrect (at 2.95 -0.6) (size 0.8 0.2) (layers "F.Cu" "F.Paste" "F.Mask") (roundrect_rratio 0.25) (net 9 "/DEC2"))
  (pad "33" smd roundrect (at 2.95 -1) (size 0.8 0.2) (layers "F.Cu" "F.Paste" "F.Mask") (roundrect_rratio 0.25) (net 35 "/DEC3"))
  (pad "34" smd roundrect (at 2.95 -1.4) (size 0.8 0.2) (layers "F.Cu" "F.Paste" "F.Mask") (roundrect_rratio 0.25) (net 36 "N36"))
  (pad "35" smd roundrect (at 2.95 -1.8) (size 0.8 0.2) (layers "F.Cu" "F.Paste" "F.Mask") (roundrect_rratio 0.25) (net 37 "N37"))
  (pad "36" smd roundrect (at 2.95 -2.2) (size 0.8 0.2) (layers "F.Cu" "F.Paste" "F.Mask") (roundrect_rratio 0.25) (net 3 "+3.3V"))
  (pad "37" smd roundrect (at 2.2 -2.95) (size 0.2 0.8) (layers "F.Cu" "F.Paste" "F.Mask") (roundrect_rratio 0.25) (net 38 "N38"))
  (pad "38" smd roundrect (at 1.8 -2.95) (size 0.2 0.8) (layers "F.Cu" "F.Paste" "F.Mask") (roundrect_rratio 0.25) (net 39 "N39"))
  (pad "39" smd roundrect (at 1.4 -2.95) (size 0.2 0.8) (layers "F.Cu" "F.Paste" "F.Mask") (roundrect_rratio 0.25) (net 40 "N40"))
  (pad "40" smd roundrect (at 1 -2.95) (size 0.2 0.8) (layers "F.Cu" "F.Paste" "F.Mask") (roundrect_rratio 0.25) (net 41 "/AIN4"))
  (pad "41" smd roundrect (at 0.6 -2.95) (size 0.2 0.8) (layers "F.Cu" "F.Paste" "F.Mask") (roundrect_rratio 0.25) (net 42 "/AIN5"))
  (pad "42" smd roundrect (at 0.2 -2.95) (size 0.2 0.8) (layers "F.Cu" "F.Paste" "F.Mask") (roundrect_rratio 0.25) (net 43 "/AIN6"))
  (pad "43" smd roundrect (at -0.2 -2.95) (size 0.2 0.8) (layers "F.Cu" "F.Paste" "F.Mask") (roundrect_rratio 0.25) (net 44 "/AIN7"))
  (pad "44" smd roundrect (at -0.6 -2.95) (size 0.2 0.8) (layers "F.Cu" "F.Paste" "F.Mask") (roundrect_rratio 0.25) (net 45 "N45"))
  (pad "45" smd roundrect (at -1 -2.95) (size 0.2 0.8) (layers "F.Cu" "F.Paste" "F.Mask") (roundrect_rratio 0.25) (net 1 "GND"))
  (pad "46" smd roundrect (at -1.4 -2.95) (size 0.2 0.8) (layers "F.Cu" "F.Paste" "F.Mask") (roundrect_rratio 0.25) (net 2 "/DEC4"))
  (pad "47" smd roundrect (at -1.8 -2.95) (size 0.2 0.8) (layers "F.Cu" "F.Paste" "F.Mask") (roundrect_rratio 0.25) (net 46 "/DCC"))
  (pad "48" smd roundrect (at -2.2 -2.95) (size 0.2 0.8) (layers "F.Cu" "F.Paste" "F.Mask") (roundrect_rratio 0.25) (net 3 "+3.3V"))
  (pad "49" smd rect (at 0 0) (size 4.6 4.6) (layers "F.Cu" "F.Mask") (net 1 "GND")))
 (gr_line (start 154.9908 82.55) (end 137.4394 82.6008) (layer "Edge.Cuts") (width 0.1))
 (gr_line (start 137.668 72.4916) (end 155.0162 72.4154) (layer "Edge.Cuts") (width 0.1))
 (gr_line (start 137.4394 82.6008) (end 137.4648 72.4662) (layer "Edge.Cuts") (width 0.1))
 (gr_line (start 137.4648 72.4662) (end 137.668 72.4916) (layer "Edge.Cuts") (width 0.1))
 (gr_line (start 155.0162 72.4154) (end 154.9908 82.55) (layer "Edge.Cuts") (width 0.1))
 (segment (start 143.822 76.54) (end 144.7038 76.54) (width 0.2) (layer "F.Cu") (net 8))
 (segment (start 143.1518 75.8698) (end 143.822 76.54) (width 0.2) (layer "F.Cu") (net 8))
 (segment (start 142.748 77.1678) (end 142.4032 77.5126) (width 0.2) (layer "F.Cu") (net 6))
 (segment (start 144.37 76.94) (end 142.9758 76.94) (width 0.2) (layer "F.Cu") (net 6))
 (segment (start 142.9758 76.94) (end 142.748 77.1678) (width 0.2) (layer "F.Cu") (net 6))
 (segment (start 142.4032 77.5126) (end 140.6274 77.5126) (width 0.2) (layer "F.Cu") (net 6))
 (segment (start 142.7226 79.149) (end 143.358 78.5136) (width 0.2) (layer "F.Cu") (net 7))
 (segment (start 143.358 77.6728) (end 143.6908 77.34) (width 0.2) (layer "F.Cu") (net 7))
 (segment (start 142.209 79.6626) (end 142.7226 79.149) (width 0.2) (layer "F.Cu") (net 7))
 (segment (start 143.6908 77.34) (end 144.37 77.34) (width 0.2) (layer "F.Cu") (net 7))
 (segment (start 140.6274 79.6626) (end 142.209 79.6626) (width 0.2) (layer "F.Cu") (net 7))
 (segment (start 143.358 78.5136) (end 143.358 77.6728) (width 0.2) (layer "F.Cu") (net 7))
 (segment (start 143.7106 74.4474) (end 144.117 74.8538) (width 0.2) (layer "F.Cu") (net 3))
 (segment (start 144.5514 74.8538) (end 145.12 75.4224) (width 0.2) (layer "F.Cu") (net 3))
 (segment (start 145.12 75.4224) (end 145.12 75.79) (width 0.2) (layer "F.Cu") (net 3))
 (segment (start 144.117 74.8538) (end 144.5514 74.8538) (width 0.2) (layer "F.Cu") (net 3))
 (segment (start 151.629175 79.8042) (end 150.764975 78.94) (width 0.2) (layer "F.Cu") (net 5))
 (segment (start 152.8674 79.8068) (end 151.793 79.8068) (width 0.2) (layer "F.Cu") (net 5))
 (segment (start 150.764975 78.94) (end 150.27 78.94) (width 0.2) (layer "F.Cu") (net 5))
 (segment (start 151.793 79.8068) (end 151.7904 79.8042) (width 0.2) (layer "F.Cu") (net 5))
 (segment (start 143.5862 73.406) (end 142.7506 74.2416) (width 0.2) (layer "F.Cu") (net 1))
 (segment (start 142.7506 75.311) (end 142.1918 75.8698) (width 0.2) (layer "F.Cu") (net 1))
 (segment (start 142.7506 74.2416) (end 142.7506 74.4474) (width 0.2) (layer "F.Cu") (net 1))
 (segment (start 153.261 77.47) (end 153.261 78.3108) (width 0.2) (layer "F.Cu") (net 1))
 (segment (start 142.7226 80.109) (end 142.7226 80.9244) (width 0.2) (layer "F.Cu") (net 1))
 (segment (start 153.261 78.3108) (end 153.2382 78.3336) (width 0.2) (layer "F.Cu") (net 1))
 (segment (start 151.859054 78.8442) (end 153.233254 77.47) (width 0.2) (layer "F.Cu") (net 1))
 (segment (start 142.7506 74.4474) (end 141.4018 74.4474) (width 0.2) (layer "F.Cu") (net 1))
 (segment (start 147.4216 78.74) (end 147.6502 78.9686) (width 0.2) (layer "F.Cu") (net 1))
 (segment (start 147.4724 78.9686) (end 146.32 77.8162) (width 0.2) (layer "F.Cu") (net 1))
 (segment (start 153.233254 77.47) (end 153.261 77.47) (width 0.2) (layer "F.Cu") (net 1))
 (segment (start 151.4862 78.54) (end 151.7904 78.8442) (width 0.2) (layer "F.Cu") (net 1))
 (segment (start 142.7506 74.4474) (end 142.7506 75.311) (width 0.2) (layer "F.Cu") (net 1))
 (segment (start 150.27 78.54) (end 151.4862 78.54) (width 0.2) (layer "F.Cu") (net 1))
 (segment (start 147.32 78.74) (end 147.4216 78.74) (width 0.2) (layer "F.Cu") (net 1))
 (segment (start 144.4524 73.406) (end 143.5862 73.406) (width 0.2) (layer "F.Cu") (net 1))
 (segment (start 153.2382 78.3336) (end 153.2382 78.6892) (width 0.2) (layer "F.Cu") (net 1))
 (segment (start 141.76 78.1278) (end 142.748 78.1278) (width 0.2) (layer "F.Cu") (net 1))
 (segment (start 146.32 75.295025) (end 146.812 74.803025) (width 0.2) (layer "F.Cu") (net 1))
 (segment (start 144.9604 73.914) (end 144.4524 73.406) (width 0.2) (layer "F.Cu") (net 1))
 (segment (start 141.4018 74.4474) (end 140.3858 74.4474) (width 0.2) (layer "F.Cu") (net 1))
 (segment (start 142.7226 81.407) (end 142.6972 81.4324) (width 0.2) (layer "F.Cu") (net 1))
 (segment (start 142.7226 80.9244) (end 142.7226 81.407) (width 0.2) (layer "F.Cu") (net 1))
 (segment (start 141.7574 78.1304) (end 141.76 78.1278) (width 0.2) (layer "F.Cu") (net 1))
 (segment (start 147.6502 78.9686) (end 147.4724 78.9686) (width 0.2) (layer "F.Cu") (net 1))
 (segment (start 147.52 78.54) (end 147.32 78.74) (width 0.2) (layer "F.Cu") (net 1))
 (segment (start 153.2382 78.6892) (end 153.2636 78.7146) (width 0.2) (layer "F.Cu") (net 1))
 (segment (start 150.27 78.54) (end 147.52 78.54) (width 0.2) (layer "F.Cu") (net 1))
 (segment (start 146.32 75.79) (end 146.32 75.295025) (width 0.2) (layer "F.Cu") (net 1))
 (segment (start 146.32 77.8162) (end 146.32 75.79) (width 0.2) (layer "F.Cu") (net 1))
 (segment (start 146.812 74.803025) (end 146.812 74.4474) (width 0.2) (layer "F.Cu") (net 1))
 (segment (start 151.7904 78.8442) (end 151.859054 78.8442) (width 0.2) (layer "F.Cu") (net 1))
 (via (at 141.7574 78.1304) (size 0.4) (drill 0.2) (layers "F.Cu" "B.Cu") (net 1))
 (via (at 153.2636 78.7146) (size 0.4) (drill 0.2) (layers "F.Cu" "B.Cu") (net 1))
 (via (at 142.6972 81.4324) (size 0.4) (drill 0.2) (layers "F.Cu" "B.Cu") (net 1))
 (via (at 140.3858 74.4474) (size 0.4) (drill 0.2) (layers "F.Cu" "B.Cu") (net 1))
 (via (at 146.812 74.4474) (size 0.4) (drill 0.2) (layers "F.Cu" "B.Cu") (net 1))
 (segment (start 152.301 77.47) (end 151.631 78.14) (width 0.2) (layer "F.Cu") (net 9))
 (segment (start 151.631 78.14) (end 150.27 78.14) (width 0.2) (layer "F.Cu") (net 9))
 (segment (start 145.9204 73.914) (end 145.9204 75.7896) (width 0.2) (layer "F.Cu") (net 2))
 (segment (start 145.9204 75.7896) (end 145.92 75.79) (width 0.2) (layer "F.Cu") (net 2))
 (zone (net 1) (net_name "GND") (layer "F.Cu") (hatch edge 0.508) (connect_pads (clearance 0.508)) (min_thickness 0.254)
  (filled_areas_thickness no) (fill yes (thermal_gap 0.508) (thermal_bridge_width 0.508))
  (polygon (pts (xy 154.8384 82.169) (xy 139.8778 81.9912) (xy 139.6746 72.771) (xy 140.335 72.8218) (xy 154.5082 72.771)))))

